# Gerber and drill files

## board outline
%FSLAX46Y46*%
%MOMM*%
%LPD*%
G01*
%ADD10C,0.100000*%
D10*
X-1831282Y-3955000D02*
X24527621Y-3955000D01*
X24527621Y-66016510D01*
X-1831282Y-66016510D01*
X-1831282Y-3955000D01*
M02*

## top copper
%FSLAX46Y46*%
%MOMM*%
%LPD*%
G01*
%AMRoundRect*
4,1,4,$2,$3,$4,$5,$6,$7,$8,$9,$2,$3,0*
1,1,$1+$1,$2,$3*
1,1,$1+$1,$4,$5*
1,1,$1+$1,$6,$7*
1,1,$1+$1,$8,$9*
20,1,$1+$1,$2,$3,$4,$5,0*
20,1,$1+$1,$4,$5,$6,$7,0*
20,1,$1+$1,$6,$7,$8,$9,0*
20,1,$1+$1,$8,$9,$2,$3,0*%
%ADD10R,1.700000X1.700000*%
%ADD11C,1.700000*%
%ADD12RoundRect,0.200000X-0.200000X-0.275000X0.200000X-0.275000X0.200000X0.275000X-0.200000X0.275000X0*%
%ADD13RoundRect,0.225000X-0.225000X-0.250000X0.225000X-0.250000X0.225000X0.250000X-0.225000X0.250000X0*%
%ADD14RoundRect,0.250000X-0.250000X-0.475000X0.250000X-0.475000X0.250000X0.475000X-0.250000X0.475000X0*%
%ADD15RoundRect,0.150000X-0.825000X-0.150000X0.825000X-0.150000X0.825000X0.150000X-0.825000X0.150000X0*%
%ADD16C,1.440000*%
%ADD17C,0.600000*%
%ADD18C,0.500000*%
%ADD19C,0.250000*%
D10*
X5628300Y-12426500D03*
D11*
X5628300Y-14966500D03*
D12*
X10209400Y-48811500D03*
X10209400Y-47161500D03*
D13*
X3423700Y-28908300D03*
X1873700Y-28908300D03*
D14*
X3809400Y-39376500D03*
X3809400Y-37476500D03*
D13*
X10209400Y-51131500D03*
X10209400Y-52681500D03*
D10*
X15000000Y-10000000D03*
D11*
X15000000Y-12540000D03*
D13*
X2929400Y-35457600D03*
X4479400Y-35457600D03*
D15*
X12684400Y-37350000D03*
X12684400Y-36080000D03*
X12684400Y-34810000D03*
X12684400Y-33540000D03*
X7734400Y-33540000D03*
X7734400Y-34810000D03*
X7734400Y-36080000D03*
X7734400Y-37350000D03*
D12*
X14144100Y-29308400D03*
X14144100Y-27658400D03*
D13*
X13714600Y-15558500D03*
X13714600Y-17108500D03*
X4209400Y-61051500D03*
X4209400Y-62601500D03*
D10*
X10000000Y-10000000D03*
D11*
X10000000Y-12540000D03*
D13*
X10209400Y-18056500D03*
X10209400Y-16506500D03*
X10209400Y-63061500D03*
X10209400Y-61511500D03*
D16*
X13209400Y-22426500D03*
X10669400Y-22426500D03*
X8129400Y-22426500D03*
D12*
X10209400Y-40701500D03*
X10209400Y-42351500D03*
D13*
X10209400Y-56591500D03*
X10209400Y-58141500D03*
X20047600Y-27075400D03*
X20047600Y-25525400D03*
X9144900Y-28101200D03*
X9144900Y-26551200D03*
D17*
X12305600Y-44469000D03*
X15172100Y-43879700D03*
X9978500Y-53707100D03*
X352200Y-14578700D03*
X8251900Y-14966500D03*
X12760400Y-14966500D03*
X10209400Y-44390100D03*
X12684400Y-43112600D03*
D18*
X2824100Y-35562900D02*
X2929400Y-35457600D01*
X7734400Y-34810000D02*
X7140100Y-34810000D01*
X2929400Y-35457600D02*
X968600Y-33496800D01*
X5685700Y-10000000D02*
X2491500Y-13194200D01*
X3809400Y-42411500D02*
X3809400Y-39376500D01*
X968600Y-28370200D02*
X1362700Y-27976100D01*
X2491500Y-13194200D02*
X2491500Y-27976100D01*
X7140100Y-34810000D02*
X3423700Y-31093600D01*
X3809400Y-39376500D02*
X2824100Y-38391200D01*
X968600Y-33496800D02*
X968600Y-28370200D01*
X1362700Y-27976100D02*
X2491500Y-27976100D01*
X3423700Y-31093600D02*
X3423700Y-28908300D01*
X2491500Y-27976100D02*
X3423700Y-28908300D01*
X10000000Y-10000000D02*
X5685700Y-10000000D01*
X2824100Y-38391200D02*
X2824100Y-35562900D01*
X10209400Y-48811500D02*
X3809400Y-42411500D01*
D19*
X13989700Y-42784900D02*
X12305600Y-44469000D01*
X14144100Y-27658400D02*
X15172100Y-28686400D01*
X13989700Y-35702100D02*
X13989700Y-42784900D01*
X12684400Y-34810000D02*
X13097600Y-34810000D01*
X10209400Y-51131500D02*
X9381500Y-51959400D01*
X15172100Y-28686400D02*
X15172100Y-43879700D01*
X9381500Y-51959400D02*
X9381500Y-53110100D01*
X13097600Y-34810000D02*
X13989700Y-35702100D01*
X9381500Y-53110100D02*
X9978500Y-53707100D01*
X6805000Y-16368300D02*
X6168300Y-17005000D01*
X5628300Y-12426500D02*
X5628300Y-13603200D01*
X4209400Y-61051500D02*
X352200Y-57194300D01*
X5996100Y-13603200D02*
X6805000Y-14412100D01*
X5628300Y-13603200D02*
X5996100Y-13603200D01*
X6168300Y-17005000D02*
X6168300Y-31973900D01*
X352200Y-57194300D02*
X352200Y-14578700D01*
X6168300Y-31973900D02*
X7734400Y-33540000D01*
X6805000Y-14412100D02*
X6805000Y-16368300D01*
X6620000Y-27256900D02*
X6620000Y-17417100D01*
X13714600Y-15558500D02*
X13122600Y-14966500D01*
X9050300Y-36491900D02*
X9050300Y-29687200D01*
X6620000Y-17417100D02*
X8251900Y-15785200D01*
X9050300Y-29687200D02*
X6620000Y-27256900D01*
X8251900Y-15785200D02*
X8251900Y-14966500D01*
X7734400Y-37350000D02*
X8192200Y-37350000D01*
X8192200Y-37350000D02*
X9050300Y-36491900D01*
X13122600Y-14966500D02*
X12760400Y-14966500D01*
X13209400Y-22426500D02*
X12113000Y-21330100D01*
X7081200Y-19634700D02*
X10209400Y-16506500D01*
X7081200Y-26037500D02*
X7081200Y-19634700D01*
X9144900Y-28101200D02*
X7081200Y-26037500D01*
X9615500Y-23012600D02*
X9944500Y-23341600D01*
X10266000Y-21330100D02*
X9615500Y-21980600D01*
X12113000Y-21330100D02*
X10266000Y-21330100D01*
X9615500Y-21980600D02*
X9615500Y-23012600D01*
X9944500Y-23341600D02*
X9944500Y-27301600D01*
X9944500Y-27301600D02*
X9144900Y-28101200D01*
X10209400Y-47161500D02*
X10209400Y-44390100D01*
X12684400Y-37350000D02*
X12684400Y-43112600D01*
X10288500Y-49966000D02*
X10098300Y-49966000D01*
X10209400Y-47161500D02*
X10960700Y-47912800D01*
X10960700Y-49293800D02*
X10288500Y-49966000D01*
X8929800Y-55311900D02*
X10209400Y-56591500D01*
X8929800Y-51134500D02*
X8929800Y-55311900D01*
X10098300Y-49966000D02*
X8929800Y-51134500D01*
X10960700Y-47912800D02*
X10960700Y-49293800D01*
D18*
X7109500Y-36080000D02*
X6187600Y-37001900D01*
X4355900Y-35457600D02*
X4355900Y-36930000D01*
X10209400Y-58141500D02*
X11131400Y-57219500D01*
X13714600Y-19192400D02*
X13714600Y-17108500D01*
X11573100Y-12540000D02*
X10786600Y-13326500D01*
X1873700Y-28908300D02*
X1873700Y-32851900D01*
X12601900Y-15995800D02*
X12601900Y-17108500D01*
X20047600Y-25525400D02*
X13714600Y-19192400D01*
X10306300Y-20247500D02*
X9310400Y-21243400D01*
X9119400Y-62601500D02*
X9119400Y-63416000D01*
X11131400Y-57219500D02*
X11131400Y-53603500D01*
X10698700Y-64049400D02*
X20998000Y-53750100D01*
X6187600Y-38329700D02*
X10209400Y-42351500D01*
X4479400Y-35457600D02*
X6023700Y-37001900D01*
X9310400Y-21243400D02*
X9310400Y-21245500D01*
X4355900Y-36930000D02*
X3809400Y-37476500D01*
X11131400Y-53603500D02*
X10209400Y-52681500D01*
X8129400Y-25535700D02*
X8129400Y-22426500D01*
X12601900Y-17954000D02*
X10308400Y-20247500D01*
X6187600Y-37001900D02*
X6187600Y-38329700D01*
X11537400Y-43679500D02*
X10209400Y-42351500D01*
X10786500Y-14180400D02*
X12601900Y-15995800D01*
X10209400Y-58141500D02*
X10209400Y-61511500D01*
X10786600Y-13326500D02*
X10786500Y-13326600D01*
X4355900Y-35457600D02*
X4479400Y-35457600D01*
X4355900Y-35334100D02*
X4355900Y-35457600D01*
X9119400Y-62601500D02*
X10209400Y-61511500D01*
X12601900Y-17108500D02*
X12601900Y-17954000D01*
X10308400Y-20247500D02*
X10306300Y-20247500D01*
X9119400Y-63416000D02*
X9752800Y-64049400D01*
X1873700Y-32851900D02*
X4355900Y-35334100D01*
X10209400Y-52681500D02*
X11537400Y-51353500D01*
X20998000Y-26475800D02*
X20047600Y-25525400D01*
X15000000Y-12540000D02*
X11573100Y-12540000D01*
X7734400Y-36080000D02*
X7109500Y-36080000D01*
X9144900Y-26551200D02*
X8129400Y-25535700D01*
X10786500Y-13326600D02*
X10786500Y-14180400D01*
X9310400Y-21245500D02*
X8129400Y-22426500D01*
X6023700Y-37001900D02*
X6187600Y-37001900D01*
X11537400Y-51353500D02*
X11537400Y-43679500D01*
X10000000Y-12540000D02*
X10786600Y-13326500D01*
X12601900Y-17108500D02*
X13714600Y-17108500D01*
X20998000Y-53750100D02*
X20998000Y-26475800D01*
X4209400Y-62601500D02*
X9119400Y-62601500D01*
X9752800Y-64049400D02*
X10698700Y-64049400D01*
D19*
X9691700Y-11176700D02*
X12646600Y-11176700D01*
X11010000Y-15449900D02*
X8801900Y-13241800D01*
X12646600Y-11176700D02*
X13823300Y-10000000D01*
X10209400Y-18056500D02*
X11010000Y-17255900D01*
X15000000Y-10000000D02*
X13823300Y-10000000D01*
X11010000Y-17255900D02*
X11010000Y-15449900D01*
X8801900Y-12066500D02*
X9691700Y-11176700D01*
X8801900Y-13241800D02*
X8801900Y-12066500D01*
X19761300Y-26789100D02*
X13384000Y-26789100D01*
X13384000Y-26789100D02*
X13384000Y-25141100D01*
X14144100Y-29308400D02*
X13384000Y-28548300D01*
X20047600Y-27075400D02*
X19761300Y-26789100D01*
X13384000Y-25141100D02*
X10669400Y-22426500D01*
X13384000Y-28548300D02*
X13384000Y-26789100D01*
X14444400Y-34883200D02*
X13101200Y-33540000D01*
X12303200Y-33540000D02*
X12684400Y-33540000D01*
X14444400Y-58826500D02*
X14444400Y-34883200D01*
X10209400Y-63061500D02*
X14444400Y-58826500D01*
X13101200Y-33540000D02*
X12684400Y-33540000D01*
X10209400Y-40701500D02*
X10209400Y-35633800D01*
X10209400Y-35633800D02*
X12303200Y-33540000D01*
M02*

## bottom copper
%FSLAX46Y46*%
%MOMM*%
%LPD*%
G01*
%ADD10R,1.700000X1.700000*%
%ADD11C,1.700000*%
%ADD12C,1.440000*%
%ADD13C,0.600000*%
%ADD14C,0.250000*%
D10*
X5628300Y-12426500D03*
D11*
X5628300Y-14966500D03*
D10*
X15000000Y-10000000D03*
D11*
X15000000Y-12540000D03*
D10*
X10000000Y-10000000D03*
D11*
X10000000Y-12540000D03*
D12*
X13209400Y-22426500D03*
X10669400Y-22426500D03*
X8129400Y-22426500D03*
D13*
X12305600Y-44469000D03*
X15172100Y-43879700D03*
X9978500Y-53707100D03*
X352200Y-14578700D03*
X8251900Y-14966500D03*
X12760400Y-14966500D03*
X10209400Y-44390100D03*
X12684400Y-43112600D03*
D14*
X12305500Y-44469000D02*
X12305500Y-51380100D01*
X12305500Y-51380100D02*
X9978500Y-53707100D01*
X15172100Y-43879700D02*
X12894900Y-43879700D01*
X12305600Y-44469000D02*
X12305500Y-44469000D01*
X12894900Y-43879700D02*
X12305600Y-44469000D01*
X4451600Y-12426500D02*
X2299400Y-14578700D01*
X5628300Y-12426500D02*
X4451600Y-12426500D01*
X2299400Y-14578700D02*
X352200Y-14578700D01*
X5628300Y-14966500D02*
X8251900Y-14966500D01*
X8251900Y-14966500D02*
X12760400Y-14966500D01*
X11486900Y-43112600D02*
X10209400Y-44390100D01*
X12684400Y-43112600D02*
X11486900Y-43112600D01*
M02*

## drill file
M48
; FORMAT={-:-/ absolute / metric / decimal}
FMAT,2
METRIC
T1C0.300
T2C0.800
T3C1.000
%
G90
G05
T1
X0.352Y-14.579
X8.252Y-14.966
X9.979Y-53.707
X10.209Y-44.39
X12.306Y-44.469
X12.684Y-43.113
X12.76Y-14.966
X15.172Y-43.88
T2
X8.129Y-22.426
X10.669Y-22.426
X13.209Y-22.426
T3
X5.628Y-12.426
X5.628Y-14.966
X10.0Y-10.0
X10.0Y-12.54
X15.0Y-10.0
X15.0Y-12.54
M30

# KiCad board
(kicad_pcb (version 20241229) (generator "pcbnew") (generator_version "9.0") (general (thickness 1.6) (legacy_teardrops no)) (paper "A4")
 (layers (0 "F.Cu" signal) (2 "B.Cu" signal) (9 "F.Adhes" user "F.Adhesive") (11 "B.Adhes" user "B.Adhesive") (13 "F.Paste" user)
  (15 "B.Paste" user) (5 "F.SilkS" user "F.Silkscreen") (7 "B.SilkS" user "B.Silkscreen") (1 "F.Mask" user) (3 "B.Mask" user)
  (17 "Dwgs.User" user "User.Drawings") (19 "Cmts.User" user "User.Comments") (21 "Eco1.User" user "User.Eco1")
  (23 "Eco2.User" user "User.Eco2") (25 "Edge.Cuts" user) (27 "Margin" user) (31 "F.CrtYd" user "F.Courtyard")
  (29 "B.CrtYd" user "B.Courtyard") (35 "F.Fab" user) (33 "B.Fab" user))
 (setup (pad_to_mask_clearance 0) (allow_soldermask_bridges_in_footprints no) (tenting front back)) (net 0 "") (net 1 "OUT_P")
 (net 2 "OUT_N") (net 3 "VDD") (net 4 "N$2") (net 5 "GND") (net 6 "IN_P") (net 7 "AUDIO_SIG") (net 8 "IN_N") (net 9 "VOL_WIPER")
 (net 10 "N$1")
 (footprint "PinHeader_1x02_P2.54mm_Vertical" (layer "F.Cu") (at 5.6283 12.4265)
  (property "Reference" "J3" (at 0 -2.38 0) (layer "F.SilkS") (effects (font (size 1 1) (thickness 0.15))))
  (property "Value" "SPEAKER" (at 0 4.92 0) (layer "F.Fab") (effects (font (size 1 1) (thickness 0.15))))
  (pad "1" thru_hole rect (at 0 0) (size 1.7 1.7) (drill 1) (layers "*.Cu" "*.Mask") (remove_unused_layers no) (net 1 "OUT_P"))
  (pad "2" thru_hole circle (at 0 2.54) (size 1.7 1.7) (drill 1) (layers "*.Cu" "*.Mask") (remove_unused_layers no) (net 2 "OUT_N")))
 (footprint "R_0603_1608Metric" (layer "F.Cu") (at 10.2094 47.9865 90)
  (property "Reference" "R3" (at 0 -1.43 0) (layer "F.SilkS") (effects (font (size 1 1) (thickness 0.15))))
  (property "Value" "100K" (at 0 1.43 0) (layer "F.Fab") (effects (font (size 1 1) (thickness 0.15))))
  (pad "1" smd roundrect (at -0.825 0) (size 0.8 0.95) (layers "F.Cu" "F.Mask" "F.Paste") (roundrect_rratio 0.25) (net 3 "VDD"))
  (pad "2" smd roundrect (at 0.825 0) (size 0.8 0.95) (layers "F.Cu" "F.Mask" "F.Paste") (roundrect_rratio 0.25) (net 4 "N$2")))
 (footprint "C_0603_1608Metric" (layer "F.Cu") (at 2.6487 28.9083 180)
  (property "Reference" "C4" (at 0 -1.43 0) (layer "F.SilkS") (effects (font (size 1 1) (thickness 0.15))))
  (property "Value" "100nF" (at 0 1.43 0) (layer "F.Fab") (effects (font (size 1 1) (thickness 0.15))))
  (pad "1" smd roundrect (at -0.775 0) (size 0.9 0.95) (layers "F.Cu" "F.Mask" "F.Paste") (roundrect_rratio 0.25) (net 3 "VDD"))
  (pad "2" smd roundrect (at 0.775 0) (size 0.9 0.95) (layers "F.Cu" "F.Mask" "F.Paste") (roundrect_rratio 0.25) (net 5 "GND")))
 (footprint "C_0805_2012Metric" (layer "F.Cu") (at 3.8094 38.4265 90)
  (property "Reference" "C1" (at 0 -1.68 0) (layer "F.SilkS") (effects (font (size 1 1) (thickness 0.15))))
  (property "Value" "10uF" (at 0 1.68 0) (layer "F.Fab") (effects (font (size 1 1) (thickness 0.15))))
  (pad "1" smd roundrect (at -0.95 0) (size 1 1.45) (layers "F.Cu" "F.Mask" "F.Paste") (roundrect_rratio 0.25) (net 3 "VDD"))
  (pad "2" smd roundrect (at 0.95 0) (size 1 1.45) (layers "F.Cu" "F.Mask" "F.Paste") (roundrect_rratio 0.25) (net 5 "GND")))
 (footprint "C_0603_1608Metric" (layer "F.Cu") (at 10.2094 51.9065 -90)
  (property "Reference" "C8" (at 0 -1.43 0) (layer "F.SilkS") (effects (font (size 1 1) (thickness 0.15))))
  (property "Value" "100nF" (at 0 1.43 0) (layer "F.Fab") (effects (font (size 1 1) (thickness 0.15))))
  (pad "1" smd roundrect (at -0.775 0) (size 0.9 0.95) (layers "F.Cu" "F.Mask" "F.Paste") (roundrect_rratio 0.25) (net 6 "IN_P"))
  (pad "2" smd roundrect (at 0.775 0) (size 0.9 0.95) (layers "F.Cu" "F.Mask" "F.Paste") (roundrect_rratio 0.25) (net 5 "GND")))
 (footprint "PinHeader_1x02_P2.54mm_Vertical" (layer "F.Cu") (at 15 10)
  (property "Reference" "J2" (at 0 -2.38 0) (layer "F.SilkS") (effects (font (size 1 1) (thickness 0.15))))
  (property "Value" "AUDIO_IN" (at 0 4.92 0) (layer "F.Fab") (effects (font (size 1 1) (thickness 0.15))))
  (pad "1" thru_hole rect (at 0 0) (size 1.7 1.7) (drill 1) (layers "*.Cu" "*.Mask") (remove_unused_layers no) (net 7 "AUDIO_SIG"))
  (pad "2" thru_hole circle (at 0 2.54) (size 1.7 1.7) (drill 1) (layers "*.Cu" "*.Mask") (remove_unused_layers no) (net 5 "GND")))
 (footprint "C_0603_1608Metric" (layer "F.Cu") (at 3.7044 35.4576)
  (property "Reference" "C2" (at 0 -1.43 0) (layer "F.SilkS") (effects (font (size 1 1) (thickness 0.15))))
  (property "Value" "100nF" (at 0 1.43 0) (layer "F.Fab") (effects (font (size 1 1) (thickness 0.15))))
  (pad "1" smd roundrect (at -0.775 0) (size 0.9 0.95) (layers "F.Cu" "F.Mask" "F.Paste") (roundrect_rratio 0.25) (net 3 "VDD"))
  (pad "2" smd roundrect (at 0.775 0) (size 0.9 0.95) (layers "F.Cu" "F.Mask" "F.Paste") (roundrect_rratio 0.25) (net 5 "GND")))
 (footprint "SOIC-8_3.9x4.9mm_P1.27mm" (layer "F.Cu") (at 10.2094 35.445 180)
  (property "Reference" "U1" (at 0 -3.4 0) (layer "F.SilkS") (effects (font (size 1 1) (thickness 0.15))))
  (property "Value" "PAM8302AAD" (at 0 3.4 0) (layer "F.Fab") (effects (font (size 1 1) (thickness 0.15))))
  (pad "1" smd roundrect (at -2.475 -1.905) (size 1.95 0.6) (layers "F.Cu" "F.Mask" "F.Paste") (roundrect_rratio 0.25) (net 4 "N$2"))
  (pad "2" smd roundrect (at -2.475 -0.635) (size 1.95 0.6) (layers "F.Cu" "F.Mask" "F.Paste") (roundrect_rratio 0.25))
  (pad "3" smd roundrect (at -2.475 0.635) (size 1.95 0.6) (layers "F.Cu" "F.Mask" "F.Paste") (roundrect_rratio 0.25) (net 6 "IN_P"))
  (pad "4" smd roundrect (at -2.475 1.905) (size 1.95 0.6) (layers "F.Cu" "F.Mask" "F.Paste") (roundrect_rratio 0.25) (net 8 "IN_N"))
  (pad "5" smd roundrect (at 2.475 1.905) (size 1.95 0.6) (layers "F.Cu" "F.Mask" "F.Paste") (roundrect_rratio 0.25) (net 1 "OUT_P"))
  (pad "6" smd roundrect (at 2.475 0.635) (size 1.95 0.6) (layers "F.Cu" "F.Mask" "F.Paste") (roundrect_rratio 0.25) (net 3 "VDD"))
  (pad "7" smd roundrect (at 2.475 -0.635) (size 1.95 0.6) (layers "F.Cu" "F.Mask" "F.Paste") (roundrect_rratio 0.25) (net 5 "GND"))
  (pad "8" smd roundrect (at 2.475 -1.905) (size 1.95 0.6) (layers "F.Cu" "F.Mask" "F.Paste") (roundrect_rratio 0.25) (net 2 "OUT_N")))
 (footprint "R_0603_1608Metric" (layer "F.Cu") (at 14.1441 28.4834 90)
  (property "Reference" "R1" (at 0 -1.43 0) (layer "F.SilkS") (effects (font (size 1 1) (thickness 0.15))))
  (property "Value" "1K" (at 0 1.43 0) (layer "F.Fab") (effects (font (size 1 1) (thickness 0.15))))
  (pad "1" smd roundrect (at -0.825 0) (size 0.8 0.95) (layers "F.Cu" "F.Mask" "F.Paste") (roundrect_rratio 0.25) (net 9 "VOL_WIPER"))
  (pad "2" smd roundrect (at 0.825 0) (size 0.8 0.95) (layers "F.Cu" "F.Mask" "F.Paste") (roundrect_rratio 0.25) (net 6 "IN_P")))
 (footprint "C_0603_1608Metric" (layer "F.Cu") (at 13.7146 16.3335 -90)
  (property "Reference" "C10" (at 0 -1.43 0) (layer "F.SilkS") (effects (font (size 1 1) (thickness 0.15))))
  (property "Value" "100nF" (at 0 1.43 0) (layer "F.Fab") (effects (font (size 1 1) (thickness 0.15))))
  (pad "1" smd roundrect (at -0.775 0) (size 0.9 0.95) (layers "F.Cu" "F.Mask" "F.Paste") (roundrect_rratio 0.25) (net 2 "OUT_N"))
  (pad "2" smd roundrect (at 0.775 0) (size 0.9 0.95) (layers "F.Cu" "F.Mask" "F.Paste") (roundrect_rratio 0.25) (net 5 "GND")))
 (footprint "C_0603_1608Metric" (layer "F.Cu") (at 4.2094 61.8265 -90)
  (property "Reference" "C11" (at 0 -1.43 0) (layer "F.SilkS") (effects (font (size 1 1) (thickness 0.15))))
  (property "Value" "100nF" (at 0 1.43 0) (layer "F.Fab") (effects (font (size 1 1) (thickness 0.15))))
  (pad "1" smd roundrect (at -0.775 0) (size 0.9 0.95) (layers "F.Cu" "F.Mask" "F.Paste") (roundrect_rratio 0.25) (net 1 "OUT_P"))
  (pad "2" smd roundrect (at 0.775 0) (size 0.9 0.95) (layers "F.Cu" "F.Mask" "F.Paste") (roundrect_rratio 0.25) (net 5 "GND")))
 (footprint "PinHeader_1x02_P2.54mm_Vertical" (layer "F.Cu") (at 10 10)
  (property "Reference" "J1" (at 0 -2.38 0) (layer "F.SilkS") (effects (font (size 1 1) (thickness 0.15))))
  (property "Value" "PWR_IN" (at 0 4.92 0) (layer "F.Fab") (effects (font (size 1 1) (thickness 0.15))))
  (pad "1" thru_hole rect (at 0 0) (size 1.7 1.7) (drill 1) (layers "*.Cu" "*.Mask") (remove_unused_layers no) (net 3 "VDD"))
  (pad "2" thru_hole circle (at 0 2.54) (size 1.7 1.7) (drill 1) (layers "*.Cu" "*.Mask") (remove_unused_layers no) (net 5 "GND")))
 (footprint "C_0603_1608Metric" (layer "F.Cu") (at 10.2094 17.2815 90)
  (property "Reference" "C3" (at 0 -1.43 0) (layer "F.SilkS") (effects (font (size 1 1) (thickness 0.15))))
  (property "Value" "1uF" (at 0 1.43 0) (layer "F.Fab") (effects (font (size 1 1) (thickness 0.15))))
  (pad "1" smd roundrect (at -0.775 0) (size 0.9 0.95) (layers "F.Cu" "F.Mask" "F.Paste") (roundrect_rratio 0.25) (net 7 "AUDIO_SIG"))
  (pad "2" smd roundrect (at 0.775 0) (size 0.9 0.95) (layers "F.Cu" "F.Mask" "F.Paste") (roundrect_rratio 0.25) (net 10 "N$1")))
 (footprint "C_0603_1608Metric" (layer "F.Cu") (at 10.2094 62.2865 90)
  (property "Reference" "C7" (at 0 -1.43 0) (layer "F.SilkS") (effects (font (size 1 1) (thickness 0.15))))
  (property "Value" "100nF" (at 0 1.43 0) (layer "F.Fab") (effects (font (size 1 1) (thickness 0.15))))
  (pad "1" smd roundrect (at -0.775 0) (size 0.9 0.95) (layers "F.Cu" "F.Mask" "F.Paste") (roundrect_rratio 0.25) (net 8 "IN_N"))
  (pad "2" smd roundrect (at 0.775 0) (size 0.9 0.95) (layers "F.Cu" "F.Mask" "F.Paste") (roundrect_rratio 0.25) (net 5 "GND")))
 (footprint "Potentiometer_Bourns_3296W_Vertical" (layer "F.Cu") (at 13.2094 22.4265)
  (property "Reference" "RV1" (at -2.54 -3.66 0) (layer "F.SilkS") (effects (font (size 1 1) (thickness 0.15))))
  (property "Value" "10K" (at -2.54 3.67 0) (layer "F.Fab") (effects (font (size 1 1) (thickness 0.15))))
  (pad "1" thru_hole circle (at 0 0) (size 1.44 1.44) (drill 0.8) (layers "*.Cu" "*.Mask") (remove_unused_layers no) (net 10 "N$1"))
  (pad "2" thru_hole circle (at -2.54 0) (size 1.44 1.44) (drill 0.8) (layers "*.Cu" "*.Mask") (remove_unused_layers no) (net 9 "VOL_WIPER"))
  (pad "3" thru_hole circle (at -5.08 0) (size 1.44 1.44) (drill 0.8) (layers "*.Cu" "*.Mask") (remove_unused_layers no) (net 5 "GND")))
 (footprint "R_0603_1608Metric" (layer "F.Cu") (at 10.2094 41.5265 -90)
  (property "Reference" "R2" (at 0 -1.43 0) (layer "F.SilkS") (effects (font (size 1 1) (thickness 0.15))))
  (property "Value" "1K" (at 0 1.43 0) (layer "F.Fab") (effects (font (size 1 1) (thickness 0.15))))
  (pad "1" smd roundrect (at -0.825 0) (size 0.8 0.95) (layers "F.Cu" "F.Mask" "F.Paste") (roundrect_rratio 0.25) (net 8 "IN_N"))
  (pad "2" smd roundrect (at 0.825 0) (size 0.8 0.95) (layers "F.Cu" "F.Mask" "F.Paste") (roundrect_rratio 0.25) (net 5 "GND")))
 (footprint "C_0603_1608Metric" (layer "F.Cu") (at 10.2094 57.3665 -90)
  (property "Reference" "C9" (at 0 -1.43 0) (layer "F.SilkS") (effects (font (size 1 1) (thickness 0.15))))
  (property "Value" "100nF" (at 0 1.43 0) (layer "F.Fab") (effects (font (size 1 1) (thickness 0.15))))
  (pad "1" smd roundrect (at -0.775 0) (size 0.9 0.95) (layers "F.Cu" "F.Mask" "F.Paste") (roundrect_rratio 0.25) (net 4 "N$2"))
  (pad "2" smd roundrect (at 0.775 0) (size 0.9 0.95) (layers "F.Cu" "F.Mask" "F.Paste") (roundrect_rratio 0.25) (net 5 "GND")))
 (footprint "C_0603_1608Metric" (layer "F.Cu") (at 20.0476 26.3004 90)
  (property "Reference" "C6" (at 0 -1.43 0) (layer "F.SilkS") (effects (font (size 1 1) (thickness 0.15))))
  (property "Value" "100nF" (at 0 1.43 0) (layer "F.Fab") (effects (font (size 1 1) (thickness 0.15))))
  (pad "1" smd roundrect (at -0.775 0) (size 0.9 0.95) (layers "F.Cu" "F.Mask" "F.Paste") (roundrect_rratio 0.25) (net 9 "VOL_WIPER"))
  (pad "2" smd roundrect (at 0.775 0) (size 0.9 0.95) (layers "F.Cu" "F.Mask" "F.Paste") (roundrect_rratio 0.25) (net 5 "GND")))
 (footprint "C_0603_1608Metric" (layer "F.Cu") (at 9.1449 27.3262 90)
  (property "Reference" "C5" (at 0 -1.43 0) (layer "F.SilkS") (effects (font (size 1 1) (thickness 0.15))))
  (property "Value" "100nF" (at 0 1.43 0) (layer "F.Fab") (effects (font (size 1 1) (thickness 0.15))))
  (pad "1" smd roundrect (at -0.775 0) (size 0.9 0.95) (layers "F.Cu" "F.Mask" "F.Paste") (roundrect_rratio 0.25) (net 10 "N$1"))
  (pad "2" smd roundrect (at 0.775 0) (size 0.9 0.95) (layers "F.Cu" "F.Mask" "F.Paste") (roundrect_rratio 0.25) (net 5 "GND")))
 (gr_rect (start -1.831282 3.955) (end 24.527621 66.01651) (stroke (width 0.1) (type solid)) (fill no) (layer "Edge.Cuts"))
 (segment (start 2.8241 35.5629) (end 2.9294 35.4576) (width 0.5) (layer "F.Cu") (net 3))
 (segment (start 7.7344 34.81) (end 7.1401 34.81) (width 0.5) (layer "F.Cu") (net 3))
 (segment (start 2.9294 35.4576) (end 0.9686 33.4968) (width 0.5) (layer "F.Cu") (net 3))
 (segment (start 5.6857 10) (end 2.4915 13.1942) (width 0.5) (layer "F.Cu") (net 3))
 (segment (start 3.8094 42.4115) (end 3.8094 39.3765) (width 0.5) (layer "F.Cu") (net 3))
 (segment (start 0.9686 28.3702) (end 1.3627 27.9761) (width 0.5) (layer "F.Cu") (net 3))
 (segment (start 2.4915 13.1942) (end 2.4915 27.9761) (width 0.5) (layer "F.Cu") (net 3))
 (segment (start 7.1401 34.81) (end 3.4237 31.0936) (width 0.5) (layer "F.Cu") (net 3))
 (segment (start 3.8094 39.3765) (end 2.8241 38.3912) (width 0.5) (layer "F.Cu") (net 3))
 (segment (start 0.9686 33.4968) (end 0.9686 28.3702) (width 0.5) (layer "F.Cu") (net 3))
 (segment (start 1.3627 27.9761) (end 2.4915 27.9761) (width 0.5) (layer "F.Cu") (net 3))
 (segment (start 3.4237 31.0936) (end 3.4237 28.9083) (width 0.5) (layer "F.Cu") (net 3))
 (segment (start 2.4915 27.9761) (end 3.4237 28.9083) (width 0.5) (layer "F.Cu") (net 3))
 (segment (start 10 10) (end 5.6857 10) (width 0.5) (layer "F.Cu") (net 3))
 (segment (start 2.8241 38.3912) (end 2.8241 35.5629) (width 0.5) (layer "F.Cu") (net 3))
 (segment (start 10.2094 48.8115) (end 3.8094 42.4115) (width 0.5) (layer "F.Cu") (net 3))
 (segment (start 13.9897 42.7849) (end 12.3056 44.469) (width 0.25) (layer "F.Cu") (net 6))
 (segment (start 14.1441 27.6584) (end 15.1721 28.6864) (width 0.25) (layer "F.Cu") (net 6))
 (segment (start 13.9897 35.7021) (end 13.9897 42.7849) (width 0.25) (layer "F.Cu") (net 6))
 (segment (start 12.6844 34.81) (end 13.0976 34.81) (width 0.25) (layer "F.Cu") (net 6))
 (segment (start 10.2094 51.1315) (end 9.3815 51.9594) (width 0.25) (layer "F.Cu") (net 6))
 (segment (start 15.1721 28.6864) (end 15.1721 43.8797) (width 0.25) (layer "F.Cu") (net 6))
 (segment (start 9.3815 51.9594) (end 9.3815 53.1101) (width 0.25) (layer "F.Cu") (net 6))
 (segment (start 13.0976 34.81) (end 13.9897 35.7021) (width 0.25) (layer "F.Cu") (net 6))
 (segment (start 9.3815 53.1101) (end 9.9785 53.7071) (width 0.25) (layer "F.Cu") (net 6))
 (via (at 12.3056 44.469) (size 0.6) (drill 0.3) (layers "F.Cu" "B.Cu") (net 6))
 (via (at 15.1721 43.8797) (size 0.6) (drill 0.3) (layers "F.Cu" "B.Cu") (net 6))
 (via (at 9.9785 53.7071) (size 0.6) (drill 0.3) (layers "F.Cu" "B.Cu") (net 6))
 (segment (start 12.3055 44.469) (end 12.3055 51.3801) (width 0.25) (layer "B.Cu") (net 6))
 (segment (start 12.3055 51.3801) (end 9.9785 53.7071) (width 0.25) (layer "B.Cu") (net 6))
 (segment (start 15.1721 43.8797) (end 12.8949 43.8797) (width 0.25) (layer "B.Cu") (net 6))
 (segment (start 12.3056 44.469) (end 12.3055 44.469) (width 0.25) (layer "B.Cu") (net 6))
 (segment (start 12.8949 43.8797) (end 12.3056 44.469) (width 0.25) (layer "B.Cu") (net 6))
 (segment (start 6.805 16.3683) (end 6.1683 17.005) (width 0.25) (layer "F.Cu") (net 1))
 (segment (start 5.6283 12.4265) (end 5.6283 13.6032) (width 0.25) (layer "F.Cu") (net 1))
 (segment (start 4.2094 61.0515) (end 0.3522 57.1943) (width 0.25) (layer "F.Cu") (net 1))
 (segment (start 5.9961 13.6032) (end 6.805 14.4121) (width 0.25) (layer "F.Cu") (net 1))
 (segment (start 5.6283 13.6032) (end 5.9961 13.6032) (width 0.25) (layer "F.Cu") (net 1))
 (segment (start 6.1683 17.005) (end 6.1683 31.9739) (width 0.25) (layer "F.Cu") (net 1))
 (segment (start 0.3522 57.1943) (end 0.3522 14.5787) (width 0.25) (layer "F.Cu") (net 1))
 (segment (start 6.1683 31.9739) (end 7.7344 33.54) (width 0.25) (layer "F.Cu") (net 1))
 (segment (start 6.805 14.4121) (end 6.805 16.3683) (width 0.25) (layer "F.Cu") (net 1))
 (via (at 0.3522 14.5787) (size 0.6) (drill 0.3) (layers "F.Cu" "B.Cu") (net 1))
 (segment (start 4.4516 12.4265) (end 2.2994 14.5787) (width 0.25) (layer "B.Cu") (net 1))
 (segment (start 5.6283 12.4265) (end 4.4516 12.4265) (width 0.25) (layer "B.Cu") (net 1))
 (segment (start 2.2994 14.5787) (end 0.3522 14.5787) (width 0.25) (layer "B.Cu") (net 1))
 (segment (start 6.62 27.2569) (end 6.62 17.4171) (width 0.25) (layer "F.Cu") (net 2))
 (segment (start 13.7146 15.5585) (end 13.1226 14.9665) (width 0.25) (layer "F.Cu") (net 2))
 (segment (start 9.0503 36.4919) (end 9.0503 29.6872) (width 0.25) (layer "F.Cu") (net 2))
 (segment (start 6.62 17.4171) (end 8.2519 15.7852) (width 0.25) (layer "F.Cu") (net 2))
 (segment (start 9.0503 29.6872) (end 6.62 27.2569) (width 0.25) (layer "F.Cu") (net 2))
 (segment (start 8.2519 15.7852) (end 8.2519 14.9665) (width 0.25) (layer "F.Cu") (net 2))
 (segment (start 7.7344 37.35) (end 8.1922 37.35) (width 0.25) (layer "F.Cu") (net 2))
 (segment (start 8.1922 37.35) (end 9.0503 36.4919) (width 0.25) (layer "F.Cu") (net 2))
 (segment (start 13.1226 14.9665) (end 12.7604 14.9665) (width 0.25) (layer "F.Cu") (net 2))
 (via (at 8.2519 14.9665) (size 0.6) (drill 0.3) (layers "F.Cu" "B.Cu") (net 2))
 (via (at 12.7604 14.9665) (size 0.6) (drill 0.3) (layers "F.Cu" "B.Cu") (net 2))
 (segment (start 5.6283 14.9665) (end 8.2519 14.9665) (width 0.25) (layer "B.Cu") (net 2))
 (segment (start 8.2519 14.9665) (end 12.7604 14.9665) (width 0.25) (layer "B.Cu") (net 2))
 (segment (start 13.2094 22.4265) (end 12.113 21.3301) (width 0.25) (layer "F.Cu") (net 10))
 (segment (start 7.0812 19.6347) (end 10.2094 16.5065) (width 0.25) (layer "F.Cu") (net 10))
 (segment (start 7.0812 26.0375) (end 7.0812 19.6347) (width 0.25) (layer "F.Cu") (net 10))
 (segment (start 9.1449 28.1012) (end 7.0812 26.0375) (width 0.25) (layer "F.Cu") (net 10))
 (segment (start 9.6155 23.0126) (end 9.9445 23.3416) (width 0.25) (layer "F.Cu") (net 10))
 (segment (start 10.266 21.3301) (end 9.6155 21.9806) (width 0.25) (layer "F.Cu") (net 10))
 (segment (start 12.113 21.3301) (end 10.266 21.3301) (width 0.25) (layer "F.Cu") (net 10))
 (segment (start 9.6155 21.9806) (end 9.6155 23.0126) (width 0.25) (layer "F.Cu") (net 10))
 (segment (start 9.9445 23.3416) (end 9.9445 27.3016) (width 0.25) (layer "F.Cu") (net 10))
 (segment (start 9.9445 27.3016) (end 9.1449 28.1012) (width 0.25) (layer "F.Cu") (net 10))
 (segment (start 10.2094 47.1615) (end 10.2094 44.3901) (width 0.25) (layer "F.Cu") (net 4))
 (segment (start 12.6844 37.35) (end 12.6844 43.1126) (width 0.25) (layer "F.Cu") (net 4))
 (segment (start 10.2885 49.966) (end 10.0983 49.966) (width 0.25) (layer "F.Cu") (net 4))
 (segment (start 10.2094 47.1615) (end 10.9607 47.9128) (width 0.25) (layer "F.Cu") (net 4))
 (segment (start 10.9607 49.2938) (end 10.2885 49.966) (width 0.25) (layer "F.Cu") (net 4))
 (segment (start 8.9298 55.3119) (end 10.2094 56.5915) (width 0.25) (layer "F.Cu") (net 4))
 (segment (start 8.9298 51.1345) (end 8.9298 55.3119) (width 0.25) (layer "F.Cu") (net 4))
 (segment (start 10.0983 49.966) (end 8.9298 51.1345) (width 0.25) (layer "F.Cu") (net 4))
 (segment (start 10.9607 47.9128) (end 10.9607 49.2938) (width 0.25) (layer "F.Cu") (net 4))
 (via (at 10.2094 44.3901) (size 0.6) (drill 0.3) (layers "F.Cu" "B.Cu") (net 4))
 (via (at 12.6844 43.1126) (size 0.6) (drill 0.3) (layers "F.Cu" "B.Cu") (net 4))
 (segment (start 11.4869 43.1126) (end 10.2094 44.3901) (width 0.25) (layer "B.Cu") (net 4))
 (segment (start 12.6844 43.1126) (end 11.4869 43.1126) (width 0.25) (layer "B.Cu") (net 4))
 (segment (start 7.1095 36.08) (end 6.1876 37.0019) (width 0.5) (layer "F.Cu") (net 5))
 (segment (start 4.3559 35.4576) (end 4.3559 36.93) (width 0.5) (layer "F.Cu") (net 5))
 (segment (start 10.2094 58.1415) (end 11.1314 57.2195) (width 0.5) (layer "F.Cu") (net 5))
 (segment (start 13.7146 19.1924) (end 13.7146 17.1085) (width 0.5) (layer "F.Cu") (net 5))
 (segment (start 11.5731 12.54) (end 10.7866 13.3265) (width 0.5) (layer "F.Cu") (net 5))
 (segment (start 1.8737 28.9083) (end 1.8737 32.8519) (width 0.5) (layer "F.Cu") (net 5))
 (segment (start 12.6019 15.9958) (end 12.6019 17.1085) (width 0.5) (layer "F.Cu") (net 5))
 (segment (start 20.0476 25.5254) (end 13.7146 19.1924) (width 0.5) (layer "F.Cu") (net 5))
 (segment (start 10.3063 20.2475) (end 9.3104 21.2434) (width 0.5) (layer "F.Cu") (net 5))
 (segment (start 9.1194 62.6015) (end 9.1194 63.416) (width 0.5) (layer "F.Cu") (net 5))
 (segment (start 11.1314 57.2195) (end 11.1314 53.6035) (width 0.5) (layer "F.Cu") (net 5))
 (segment (start 10.6987 64.0494) (end 20.998 53.7501) (width 0.5) (layer "F.Cu") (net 5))
 (segment (start 6.1876 38.3297) (end 10.2094 42.3515) (width 0.5) (layer "F.Cu") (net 5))
 (segment (start 4.4794 35.4576) (end 6.0237 37.0019) (width 0.5) (layer "F.Cu") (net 5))
 (segment (start 9.3104 21.2434) (end 9.3104 21.2455) (width 0.5) (layer "F.Cu") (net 5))
 (segment (start 4.3559 36.93) (end 3.8094 37.4765) (width 0.5) (layer "F.Cu") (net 5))
 (segment (start 11.1314 53.6035) (end 10.2094 52.6815) (width 0.5) (layer "F.Cu") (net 5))
 (segment (start 8.1294 25.5357) (end 8.1294 22.4265) (width 0.5) (layer "F.Cu") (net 5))
 (segment (start 12.6019 17.954) (end 10.3084 20.2475) (width 0.5) (layer "F.Cu") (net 5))
 (segment (start 6.1876 37.0019) (end 6.1876 38.3297) (width 0.5) (layer "F.Cu") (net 5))
 (segment (start 11.5374 43.6795) (end 10.2094 42.3515) (width 0.5) (layer "F.Cu") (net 5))
 (segment (start 10.7865 14.1804) (end 12.6019 15.9958) (width 0.5) (layer "F.Cu") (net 5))
 (segment (start 10.2094 58.1415) (end 10.2094 61.5115) (width 0.5) (layer "F.Cu") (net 5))
 (segment (start 10.7866 13.3265) (end 10.7865 13.3266) (width 0.5) (layer "F.Cu") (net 5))
 (segment (start 4.3559 35.4576) (end 4.4794 35.4576) (width 0.5) (layer "F.Cu") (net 5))
 (segment (start 4.3559 35.3341) (end 4.3559 35.4576) (width 0.5) (layer "F.Cu") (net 5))
 (segment (start 9.1194 62.6015) (end 10.2094 61.5115) (width 0.5) (layer "F.Cu") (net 5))
 (segment (start 12.6019 17.1085) (end 12.6019 17.954) (width 0.5) (layer "F.Cu") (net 5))
 (segment (start 10.3084 20.2475) (end 10.3063 20.2475) (width 0.5) (layer "F.Cu") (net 5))
 (segment (start 9.1194 63.416) (end 9.7528 64.0494) (width 0.5) (layer "F.Cu") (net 5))
 (segment (start 1.8737 32.8519) (end 4.3559 35.3341) (width 0.5) (layer "F.Cu") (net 5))
 (segment (start 10.2094 52.6815) (end 11.5374 51.3535) (width 0.5) (layer "F.Cu") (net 5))
 (segment (start 20.998 26.4758) (end 20.0476 25.5254) (width 0.5) (layer "F.Cu") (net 5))
 (segment (start 15 12.54) (end 11.5731 12.54) (width 0.5) (layer "F.Cu") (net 5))
 (segment (start 7.7344 36.08) (end 7.1095 36.08) (width 0.5) (layer "F.Cu") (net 5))
 (segment (start 9.1449 26.5512) (end 8.1294 25.5357) (width 0.5) (layer "F.Cu") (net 5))
 (segment (start 10.7865 13.3266) (end 10.7865 14.1804) (width 0.5) (layer "F.Cu") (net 5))
 (segment (start 9.3104 21.2455) (end 8.1294 22.4265) (width 0.5) (layer "F.Cu") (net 5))
 (segment (start 6.0237 37.0019) (end 6.1876 37.0019) (width 0.5) (layer "F.Cu") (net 5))
 (segment (start 11.5374 51.3535) (end 11.5374 43.6795) (width 0.5) (layer "F.Cu") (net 5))
 (segment (start 10 12.54) (end 10.7866 13.3265) (width 0.5) (layer "F.Cu") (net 5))
 (segment (start 12.6019 17.1085) (end 13.7146 17.1085) (width 0.5) (layer "F.Cu") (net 5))
 (segment (start 20.998 53.7501) (end 20.998 26.4758) (width 0.5) (layer "F.Cu") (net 5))
 (segment (start 4.2094 62.6015) (end 9.1194 62.6015) (width 0.5) (layer "F.Cu") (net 5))
 (segment (start 9.7528 64.0494) (end 10.6987 64.0494) (width 0.5) (layer "F.Cu") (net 5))
 (segment (start 9.6917 11.1767) (end 12.6466 11.1767) (width 0.25) (layer "F.Cu") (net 7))
 (segment (start 11.01 15.4499) (end 8.8019 13.2418) (width 0.25) (layer "F.Cu") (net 7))
 (segment (start 12.6466 11.1767) (end 13.8233 10) (width 0.25) (layer "F.Cu") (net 7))
 (segment (start 10.2094 18.0565) (end 11.01 17.2559) (width 0.25) (layer "F.Cu") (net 7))
 (segment (start 15 10) (end 13.8233 10) (width 0.25) (layer "F.Cu") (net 7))
 (segment (start 11.01 17.2559) (end 11.01 15.4499) (width 0.25) (layer "F.Cu") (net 7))
 (segment (start 8.8019 12.0665) (end 9.6917 11.1767) (width 0.25) (layer "F.Cu") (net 7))
 (segment (start 8.8019 13.2418) (end 8.8019 12.0665) (width 0.25) (layer "F.Cu") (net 7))
 (segment (start 19.7613 26.7891) (end 13.384 26.7891) (width 0.25) (layer "F.Cu") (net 9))
 (segment (start 13.384 26.7891) (end 13.384 25.1411) (width 0.25) (layer "F.Cu") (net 9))
 (segment (start 14.1441 29.3084) (end 13.384 28.5483) (width 0.25) (layer "F.Cu") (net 9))
 (segment (start 20.0476 27.0754) (end 19.7613 26.7891) (width 0.25) (layer "F.Cu") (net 9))
 (segment (start 13.384 25.1411) (end 10.6694 22.4265) (width 0.25) (layer "F.Cu") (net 9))
 (segment (start 13.384 28.5483) (end 13.384 26.7891) (width 0.25) (layer "F.Cu") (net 9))
 (segment (start 14.4444 34.8832) (end 13.1012 33.54) (width 0.25) (layer "F.Cu") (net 8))
 (segment (start 12.3032 33.54) (end 12.6844 33.54) (width 0.25) (layer "F.Cu") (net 8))
 (segment (start 14.4444 58.8265) (end 14.4444 34.8832) (width 0.25) (layer "F.Cu") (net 8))
 (segment (start 10.2094 63.0615) (end 14.4444 58.8265) (width 0.25) (layer "F.Cu") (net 8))
 (segment (start 13.1012 33.54) (end 12.6844 33.54) (width 0.25) (layer "F.Cu") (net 8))
 (segment (start 10.2094 40.7015) (end 10.2094 35.6338) (width 0.25) (layer "F.Cu") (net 8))
 (segment (start 10.2094 35.6338) (end 12.3032 33.54) (width 0.25) (layer "F.Cu") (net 8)))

